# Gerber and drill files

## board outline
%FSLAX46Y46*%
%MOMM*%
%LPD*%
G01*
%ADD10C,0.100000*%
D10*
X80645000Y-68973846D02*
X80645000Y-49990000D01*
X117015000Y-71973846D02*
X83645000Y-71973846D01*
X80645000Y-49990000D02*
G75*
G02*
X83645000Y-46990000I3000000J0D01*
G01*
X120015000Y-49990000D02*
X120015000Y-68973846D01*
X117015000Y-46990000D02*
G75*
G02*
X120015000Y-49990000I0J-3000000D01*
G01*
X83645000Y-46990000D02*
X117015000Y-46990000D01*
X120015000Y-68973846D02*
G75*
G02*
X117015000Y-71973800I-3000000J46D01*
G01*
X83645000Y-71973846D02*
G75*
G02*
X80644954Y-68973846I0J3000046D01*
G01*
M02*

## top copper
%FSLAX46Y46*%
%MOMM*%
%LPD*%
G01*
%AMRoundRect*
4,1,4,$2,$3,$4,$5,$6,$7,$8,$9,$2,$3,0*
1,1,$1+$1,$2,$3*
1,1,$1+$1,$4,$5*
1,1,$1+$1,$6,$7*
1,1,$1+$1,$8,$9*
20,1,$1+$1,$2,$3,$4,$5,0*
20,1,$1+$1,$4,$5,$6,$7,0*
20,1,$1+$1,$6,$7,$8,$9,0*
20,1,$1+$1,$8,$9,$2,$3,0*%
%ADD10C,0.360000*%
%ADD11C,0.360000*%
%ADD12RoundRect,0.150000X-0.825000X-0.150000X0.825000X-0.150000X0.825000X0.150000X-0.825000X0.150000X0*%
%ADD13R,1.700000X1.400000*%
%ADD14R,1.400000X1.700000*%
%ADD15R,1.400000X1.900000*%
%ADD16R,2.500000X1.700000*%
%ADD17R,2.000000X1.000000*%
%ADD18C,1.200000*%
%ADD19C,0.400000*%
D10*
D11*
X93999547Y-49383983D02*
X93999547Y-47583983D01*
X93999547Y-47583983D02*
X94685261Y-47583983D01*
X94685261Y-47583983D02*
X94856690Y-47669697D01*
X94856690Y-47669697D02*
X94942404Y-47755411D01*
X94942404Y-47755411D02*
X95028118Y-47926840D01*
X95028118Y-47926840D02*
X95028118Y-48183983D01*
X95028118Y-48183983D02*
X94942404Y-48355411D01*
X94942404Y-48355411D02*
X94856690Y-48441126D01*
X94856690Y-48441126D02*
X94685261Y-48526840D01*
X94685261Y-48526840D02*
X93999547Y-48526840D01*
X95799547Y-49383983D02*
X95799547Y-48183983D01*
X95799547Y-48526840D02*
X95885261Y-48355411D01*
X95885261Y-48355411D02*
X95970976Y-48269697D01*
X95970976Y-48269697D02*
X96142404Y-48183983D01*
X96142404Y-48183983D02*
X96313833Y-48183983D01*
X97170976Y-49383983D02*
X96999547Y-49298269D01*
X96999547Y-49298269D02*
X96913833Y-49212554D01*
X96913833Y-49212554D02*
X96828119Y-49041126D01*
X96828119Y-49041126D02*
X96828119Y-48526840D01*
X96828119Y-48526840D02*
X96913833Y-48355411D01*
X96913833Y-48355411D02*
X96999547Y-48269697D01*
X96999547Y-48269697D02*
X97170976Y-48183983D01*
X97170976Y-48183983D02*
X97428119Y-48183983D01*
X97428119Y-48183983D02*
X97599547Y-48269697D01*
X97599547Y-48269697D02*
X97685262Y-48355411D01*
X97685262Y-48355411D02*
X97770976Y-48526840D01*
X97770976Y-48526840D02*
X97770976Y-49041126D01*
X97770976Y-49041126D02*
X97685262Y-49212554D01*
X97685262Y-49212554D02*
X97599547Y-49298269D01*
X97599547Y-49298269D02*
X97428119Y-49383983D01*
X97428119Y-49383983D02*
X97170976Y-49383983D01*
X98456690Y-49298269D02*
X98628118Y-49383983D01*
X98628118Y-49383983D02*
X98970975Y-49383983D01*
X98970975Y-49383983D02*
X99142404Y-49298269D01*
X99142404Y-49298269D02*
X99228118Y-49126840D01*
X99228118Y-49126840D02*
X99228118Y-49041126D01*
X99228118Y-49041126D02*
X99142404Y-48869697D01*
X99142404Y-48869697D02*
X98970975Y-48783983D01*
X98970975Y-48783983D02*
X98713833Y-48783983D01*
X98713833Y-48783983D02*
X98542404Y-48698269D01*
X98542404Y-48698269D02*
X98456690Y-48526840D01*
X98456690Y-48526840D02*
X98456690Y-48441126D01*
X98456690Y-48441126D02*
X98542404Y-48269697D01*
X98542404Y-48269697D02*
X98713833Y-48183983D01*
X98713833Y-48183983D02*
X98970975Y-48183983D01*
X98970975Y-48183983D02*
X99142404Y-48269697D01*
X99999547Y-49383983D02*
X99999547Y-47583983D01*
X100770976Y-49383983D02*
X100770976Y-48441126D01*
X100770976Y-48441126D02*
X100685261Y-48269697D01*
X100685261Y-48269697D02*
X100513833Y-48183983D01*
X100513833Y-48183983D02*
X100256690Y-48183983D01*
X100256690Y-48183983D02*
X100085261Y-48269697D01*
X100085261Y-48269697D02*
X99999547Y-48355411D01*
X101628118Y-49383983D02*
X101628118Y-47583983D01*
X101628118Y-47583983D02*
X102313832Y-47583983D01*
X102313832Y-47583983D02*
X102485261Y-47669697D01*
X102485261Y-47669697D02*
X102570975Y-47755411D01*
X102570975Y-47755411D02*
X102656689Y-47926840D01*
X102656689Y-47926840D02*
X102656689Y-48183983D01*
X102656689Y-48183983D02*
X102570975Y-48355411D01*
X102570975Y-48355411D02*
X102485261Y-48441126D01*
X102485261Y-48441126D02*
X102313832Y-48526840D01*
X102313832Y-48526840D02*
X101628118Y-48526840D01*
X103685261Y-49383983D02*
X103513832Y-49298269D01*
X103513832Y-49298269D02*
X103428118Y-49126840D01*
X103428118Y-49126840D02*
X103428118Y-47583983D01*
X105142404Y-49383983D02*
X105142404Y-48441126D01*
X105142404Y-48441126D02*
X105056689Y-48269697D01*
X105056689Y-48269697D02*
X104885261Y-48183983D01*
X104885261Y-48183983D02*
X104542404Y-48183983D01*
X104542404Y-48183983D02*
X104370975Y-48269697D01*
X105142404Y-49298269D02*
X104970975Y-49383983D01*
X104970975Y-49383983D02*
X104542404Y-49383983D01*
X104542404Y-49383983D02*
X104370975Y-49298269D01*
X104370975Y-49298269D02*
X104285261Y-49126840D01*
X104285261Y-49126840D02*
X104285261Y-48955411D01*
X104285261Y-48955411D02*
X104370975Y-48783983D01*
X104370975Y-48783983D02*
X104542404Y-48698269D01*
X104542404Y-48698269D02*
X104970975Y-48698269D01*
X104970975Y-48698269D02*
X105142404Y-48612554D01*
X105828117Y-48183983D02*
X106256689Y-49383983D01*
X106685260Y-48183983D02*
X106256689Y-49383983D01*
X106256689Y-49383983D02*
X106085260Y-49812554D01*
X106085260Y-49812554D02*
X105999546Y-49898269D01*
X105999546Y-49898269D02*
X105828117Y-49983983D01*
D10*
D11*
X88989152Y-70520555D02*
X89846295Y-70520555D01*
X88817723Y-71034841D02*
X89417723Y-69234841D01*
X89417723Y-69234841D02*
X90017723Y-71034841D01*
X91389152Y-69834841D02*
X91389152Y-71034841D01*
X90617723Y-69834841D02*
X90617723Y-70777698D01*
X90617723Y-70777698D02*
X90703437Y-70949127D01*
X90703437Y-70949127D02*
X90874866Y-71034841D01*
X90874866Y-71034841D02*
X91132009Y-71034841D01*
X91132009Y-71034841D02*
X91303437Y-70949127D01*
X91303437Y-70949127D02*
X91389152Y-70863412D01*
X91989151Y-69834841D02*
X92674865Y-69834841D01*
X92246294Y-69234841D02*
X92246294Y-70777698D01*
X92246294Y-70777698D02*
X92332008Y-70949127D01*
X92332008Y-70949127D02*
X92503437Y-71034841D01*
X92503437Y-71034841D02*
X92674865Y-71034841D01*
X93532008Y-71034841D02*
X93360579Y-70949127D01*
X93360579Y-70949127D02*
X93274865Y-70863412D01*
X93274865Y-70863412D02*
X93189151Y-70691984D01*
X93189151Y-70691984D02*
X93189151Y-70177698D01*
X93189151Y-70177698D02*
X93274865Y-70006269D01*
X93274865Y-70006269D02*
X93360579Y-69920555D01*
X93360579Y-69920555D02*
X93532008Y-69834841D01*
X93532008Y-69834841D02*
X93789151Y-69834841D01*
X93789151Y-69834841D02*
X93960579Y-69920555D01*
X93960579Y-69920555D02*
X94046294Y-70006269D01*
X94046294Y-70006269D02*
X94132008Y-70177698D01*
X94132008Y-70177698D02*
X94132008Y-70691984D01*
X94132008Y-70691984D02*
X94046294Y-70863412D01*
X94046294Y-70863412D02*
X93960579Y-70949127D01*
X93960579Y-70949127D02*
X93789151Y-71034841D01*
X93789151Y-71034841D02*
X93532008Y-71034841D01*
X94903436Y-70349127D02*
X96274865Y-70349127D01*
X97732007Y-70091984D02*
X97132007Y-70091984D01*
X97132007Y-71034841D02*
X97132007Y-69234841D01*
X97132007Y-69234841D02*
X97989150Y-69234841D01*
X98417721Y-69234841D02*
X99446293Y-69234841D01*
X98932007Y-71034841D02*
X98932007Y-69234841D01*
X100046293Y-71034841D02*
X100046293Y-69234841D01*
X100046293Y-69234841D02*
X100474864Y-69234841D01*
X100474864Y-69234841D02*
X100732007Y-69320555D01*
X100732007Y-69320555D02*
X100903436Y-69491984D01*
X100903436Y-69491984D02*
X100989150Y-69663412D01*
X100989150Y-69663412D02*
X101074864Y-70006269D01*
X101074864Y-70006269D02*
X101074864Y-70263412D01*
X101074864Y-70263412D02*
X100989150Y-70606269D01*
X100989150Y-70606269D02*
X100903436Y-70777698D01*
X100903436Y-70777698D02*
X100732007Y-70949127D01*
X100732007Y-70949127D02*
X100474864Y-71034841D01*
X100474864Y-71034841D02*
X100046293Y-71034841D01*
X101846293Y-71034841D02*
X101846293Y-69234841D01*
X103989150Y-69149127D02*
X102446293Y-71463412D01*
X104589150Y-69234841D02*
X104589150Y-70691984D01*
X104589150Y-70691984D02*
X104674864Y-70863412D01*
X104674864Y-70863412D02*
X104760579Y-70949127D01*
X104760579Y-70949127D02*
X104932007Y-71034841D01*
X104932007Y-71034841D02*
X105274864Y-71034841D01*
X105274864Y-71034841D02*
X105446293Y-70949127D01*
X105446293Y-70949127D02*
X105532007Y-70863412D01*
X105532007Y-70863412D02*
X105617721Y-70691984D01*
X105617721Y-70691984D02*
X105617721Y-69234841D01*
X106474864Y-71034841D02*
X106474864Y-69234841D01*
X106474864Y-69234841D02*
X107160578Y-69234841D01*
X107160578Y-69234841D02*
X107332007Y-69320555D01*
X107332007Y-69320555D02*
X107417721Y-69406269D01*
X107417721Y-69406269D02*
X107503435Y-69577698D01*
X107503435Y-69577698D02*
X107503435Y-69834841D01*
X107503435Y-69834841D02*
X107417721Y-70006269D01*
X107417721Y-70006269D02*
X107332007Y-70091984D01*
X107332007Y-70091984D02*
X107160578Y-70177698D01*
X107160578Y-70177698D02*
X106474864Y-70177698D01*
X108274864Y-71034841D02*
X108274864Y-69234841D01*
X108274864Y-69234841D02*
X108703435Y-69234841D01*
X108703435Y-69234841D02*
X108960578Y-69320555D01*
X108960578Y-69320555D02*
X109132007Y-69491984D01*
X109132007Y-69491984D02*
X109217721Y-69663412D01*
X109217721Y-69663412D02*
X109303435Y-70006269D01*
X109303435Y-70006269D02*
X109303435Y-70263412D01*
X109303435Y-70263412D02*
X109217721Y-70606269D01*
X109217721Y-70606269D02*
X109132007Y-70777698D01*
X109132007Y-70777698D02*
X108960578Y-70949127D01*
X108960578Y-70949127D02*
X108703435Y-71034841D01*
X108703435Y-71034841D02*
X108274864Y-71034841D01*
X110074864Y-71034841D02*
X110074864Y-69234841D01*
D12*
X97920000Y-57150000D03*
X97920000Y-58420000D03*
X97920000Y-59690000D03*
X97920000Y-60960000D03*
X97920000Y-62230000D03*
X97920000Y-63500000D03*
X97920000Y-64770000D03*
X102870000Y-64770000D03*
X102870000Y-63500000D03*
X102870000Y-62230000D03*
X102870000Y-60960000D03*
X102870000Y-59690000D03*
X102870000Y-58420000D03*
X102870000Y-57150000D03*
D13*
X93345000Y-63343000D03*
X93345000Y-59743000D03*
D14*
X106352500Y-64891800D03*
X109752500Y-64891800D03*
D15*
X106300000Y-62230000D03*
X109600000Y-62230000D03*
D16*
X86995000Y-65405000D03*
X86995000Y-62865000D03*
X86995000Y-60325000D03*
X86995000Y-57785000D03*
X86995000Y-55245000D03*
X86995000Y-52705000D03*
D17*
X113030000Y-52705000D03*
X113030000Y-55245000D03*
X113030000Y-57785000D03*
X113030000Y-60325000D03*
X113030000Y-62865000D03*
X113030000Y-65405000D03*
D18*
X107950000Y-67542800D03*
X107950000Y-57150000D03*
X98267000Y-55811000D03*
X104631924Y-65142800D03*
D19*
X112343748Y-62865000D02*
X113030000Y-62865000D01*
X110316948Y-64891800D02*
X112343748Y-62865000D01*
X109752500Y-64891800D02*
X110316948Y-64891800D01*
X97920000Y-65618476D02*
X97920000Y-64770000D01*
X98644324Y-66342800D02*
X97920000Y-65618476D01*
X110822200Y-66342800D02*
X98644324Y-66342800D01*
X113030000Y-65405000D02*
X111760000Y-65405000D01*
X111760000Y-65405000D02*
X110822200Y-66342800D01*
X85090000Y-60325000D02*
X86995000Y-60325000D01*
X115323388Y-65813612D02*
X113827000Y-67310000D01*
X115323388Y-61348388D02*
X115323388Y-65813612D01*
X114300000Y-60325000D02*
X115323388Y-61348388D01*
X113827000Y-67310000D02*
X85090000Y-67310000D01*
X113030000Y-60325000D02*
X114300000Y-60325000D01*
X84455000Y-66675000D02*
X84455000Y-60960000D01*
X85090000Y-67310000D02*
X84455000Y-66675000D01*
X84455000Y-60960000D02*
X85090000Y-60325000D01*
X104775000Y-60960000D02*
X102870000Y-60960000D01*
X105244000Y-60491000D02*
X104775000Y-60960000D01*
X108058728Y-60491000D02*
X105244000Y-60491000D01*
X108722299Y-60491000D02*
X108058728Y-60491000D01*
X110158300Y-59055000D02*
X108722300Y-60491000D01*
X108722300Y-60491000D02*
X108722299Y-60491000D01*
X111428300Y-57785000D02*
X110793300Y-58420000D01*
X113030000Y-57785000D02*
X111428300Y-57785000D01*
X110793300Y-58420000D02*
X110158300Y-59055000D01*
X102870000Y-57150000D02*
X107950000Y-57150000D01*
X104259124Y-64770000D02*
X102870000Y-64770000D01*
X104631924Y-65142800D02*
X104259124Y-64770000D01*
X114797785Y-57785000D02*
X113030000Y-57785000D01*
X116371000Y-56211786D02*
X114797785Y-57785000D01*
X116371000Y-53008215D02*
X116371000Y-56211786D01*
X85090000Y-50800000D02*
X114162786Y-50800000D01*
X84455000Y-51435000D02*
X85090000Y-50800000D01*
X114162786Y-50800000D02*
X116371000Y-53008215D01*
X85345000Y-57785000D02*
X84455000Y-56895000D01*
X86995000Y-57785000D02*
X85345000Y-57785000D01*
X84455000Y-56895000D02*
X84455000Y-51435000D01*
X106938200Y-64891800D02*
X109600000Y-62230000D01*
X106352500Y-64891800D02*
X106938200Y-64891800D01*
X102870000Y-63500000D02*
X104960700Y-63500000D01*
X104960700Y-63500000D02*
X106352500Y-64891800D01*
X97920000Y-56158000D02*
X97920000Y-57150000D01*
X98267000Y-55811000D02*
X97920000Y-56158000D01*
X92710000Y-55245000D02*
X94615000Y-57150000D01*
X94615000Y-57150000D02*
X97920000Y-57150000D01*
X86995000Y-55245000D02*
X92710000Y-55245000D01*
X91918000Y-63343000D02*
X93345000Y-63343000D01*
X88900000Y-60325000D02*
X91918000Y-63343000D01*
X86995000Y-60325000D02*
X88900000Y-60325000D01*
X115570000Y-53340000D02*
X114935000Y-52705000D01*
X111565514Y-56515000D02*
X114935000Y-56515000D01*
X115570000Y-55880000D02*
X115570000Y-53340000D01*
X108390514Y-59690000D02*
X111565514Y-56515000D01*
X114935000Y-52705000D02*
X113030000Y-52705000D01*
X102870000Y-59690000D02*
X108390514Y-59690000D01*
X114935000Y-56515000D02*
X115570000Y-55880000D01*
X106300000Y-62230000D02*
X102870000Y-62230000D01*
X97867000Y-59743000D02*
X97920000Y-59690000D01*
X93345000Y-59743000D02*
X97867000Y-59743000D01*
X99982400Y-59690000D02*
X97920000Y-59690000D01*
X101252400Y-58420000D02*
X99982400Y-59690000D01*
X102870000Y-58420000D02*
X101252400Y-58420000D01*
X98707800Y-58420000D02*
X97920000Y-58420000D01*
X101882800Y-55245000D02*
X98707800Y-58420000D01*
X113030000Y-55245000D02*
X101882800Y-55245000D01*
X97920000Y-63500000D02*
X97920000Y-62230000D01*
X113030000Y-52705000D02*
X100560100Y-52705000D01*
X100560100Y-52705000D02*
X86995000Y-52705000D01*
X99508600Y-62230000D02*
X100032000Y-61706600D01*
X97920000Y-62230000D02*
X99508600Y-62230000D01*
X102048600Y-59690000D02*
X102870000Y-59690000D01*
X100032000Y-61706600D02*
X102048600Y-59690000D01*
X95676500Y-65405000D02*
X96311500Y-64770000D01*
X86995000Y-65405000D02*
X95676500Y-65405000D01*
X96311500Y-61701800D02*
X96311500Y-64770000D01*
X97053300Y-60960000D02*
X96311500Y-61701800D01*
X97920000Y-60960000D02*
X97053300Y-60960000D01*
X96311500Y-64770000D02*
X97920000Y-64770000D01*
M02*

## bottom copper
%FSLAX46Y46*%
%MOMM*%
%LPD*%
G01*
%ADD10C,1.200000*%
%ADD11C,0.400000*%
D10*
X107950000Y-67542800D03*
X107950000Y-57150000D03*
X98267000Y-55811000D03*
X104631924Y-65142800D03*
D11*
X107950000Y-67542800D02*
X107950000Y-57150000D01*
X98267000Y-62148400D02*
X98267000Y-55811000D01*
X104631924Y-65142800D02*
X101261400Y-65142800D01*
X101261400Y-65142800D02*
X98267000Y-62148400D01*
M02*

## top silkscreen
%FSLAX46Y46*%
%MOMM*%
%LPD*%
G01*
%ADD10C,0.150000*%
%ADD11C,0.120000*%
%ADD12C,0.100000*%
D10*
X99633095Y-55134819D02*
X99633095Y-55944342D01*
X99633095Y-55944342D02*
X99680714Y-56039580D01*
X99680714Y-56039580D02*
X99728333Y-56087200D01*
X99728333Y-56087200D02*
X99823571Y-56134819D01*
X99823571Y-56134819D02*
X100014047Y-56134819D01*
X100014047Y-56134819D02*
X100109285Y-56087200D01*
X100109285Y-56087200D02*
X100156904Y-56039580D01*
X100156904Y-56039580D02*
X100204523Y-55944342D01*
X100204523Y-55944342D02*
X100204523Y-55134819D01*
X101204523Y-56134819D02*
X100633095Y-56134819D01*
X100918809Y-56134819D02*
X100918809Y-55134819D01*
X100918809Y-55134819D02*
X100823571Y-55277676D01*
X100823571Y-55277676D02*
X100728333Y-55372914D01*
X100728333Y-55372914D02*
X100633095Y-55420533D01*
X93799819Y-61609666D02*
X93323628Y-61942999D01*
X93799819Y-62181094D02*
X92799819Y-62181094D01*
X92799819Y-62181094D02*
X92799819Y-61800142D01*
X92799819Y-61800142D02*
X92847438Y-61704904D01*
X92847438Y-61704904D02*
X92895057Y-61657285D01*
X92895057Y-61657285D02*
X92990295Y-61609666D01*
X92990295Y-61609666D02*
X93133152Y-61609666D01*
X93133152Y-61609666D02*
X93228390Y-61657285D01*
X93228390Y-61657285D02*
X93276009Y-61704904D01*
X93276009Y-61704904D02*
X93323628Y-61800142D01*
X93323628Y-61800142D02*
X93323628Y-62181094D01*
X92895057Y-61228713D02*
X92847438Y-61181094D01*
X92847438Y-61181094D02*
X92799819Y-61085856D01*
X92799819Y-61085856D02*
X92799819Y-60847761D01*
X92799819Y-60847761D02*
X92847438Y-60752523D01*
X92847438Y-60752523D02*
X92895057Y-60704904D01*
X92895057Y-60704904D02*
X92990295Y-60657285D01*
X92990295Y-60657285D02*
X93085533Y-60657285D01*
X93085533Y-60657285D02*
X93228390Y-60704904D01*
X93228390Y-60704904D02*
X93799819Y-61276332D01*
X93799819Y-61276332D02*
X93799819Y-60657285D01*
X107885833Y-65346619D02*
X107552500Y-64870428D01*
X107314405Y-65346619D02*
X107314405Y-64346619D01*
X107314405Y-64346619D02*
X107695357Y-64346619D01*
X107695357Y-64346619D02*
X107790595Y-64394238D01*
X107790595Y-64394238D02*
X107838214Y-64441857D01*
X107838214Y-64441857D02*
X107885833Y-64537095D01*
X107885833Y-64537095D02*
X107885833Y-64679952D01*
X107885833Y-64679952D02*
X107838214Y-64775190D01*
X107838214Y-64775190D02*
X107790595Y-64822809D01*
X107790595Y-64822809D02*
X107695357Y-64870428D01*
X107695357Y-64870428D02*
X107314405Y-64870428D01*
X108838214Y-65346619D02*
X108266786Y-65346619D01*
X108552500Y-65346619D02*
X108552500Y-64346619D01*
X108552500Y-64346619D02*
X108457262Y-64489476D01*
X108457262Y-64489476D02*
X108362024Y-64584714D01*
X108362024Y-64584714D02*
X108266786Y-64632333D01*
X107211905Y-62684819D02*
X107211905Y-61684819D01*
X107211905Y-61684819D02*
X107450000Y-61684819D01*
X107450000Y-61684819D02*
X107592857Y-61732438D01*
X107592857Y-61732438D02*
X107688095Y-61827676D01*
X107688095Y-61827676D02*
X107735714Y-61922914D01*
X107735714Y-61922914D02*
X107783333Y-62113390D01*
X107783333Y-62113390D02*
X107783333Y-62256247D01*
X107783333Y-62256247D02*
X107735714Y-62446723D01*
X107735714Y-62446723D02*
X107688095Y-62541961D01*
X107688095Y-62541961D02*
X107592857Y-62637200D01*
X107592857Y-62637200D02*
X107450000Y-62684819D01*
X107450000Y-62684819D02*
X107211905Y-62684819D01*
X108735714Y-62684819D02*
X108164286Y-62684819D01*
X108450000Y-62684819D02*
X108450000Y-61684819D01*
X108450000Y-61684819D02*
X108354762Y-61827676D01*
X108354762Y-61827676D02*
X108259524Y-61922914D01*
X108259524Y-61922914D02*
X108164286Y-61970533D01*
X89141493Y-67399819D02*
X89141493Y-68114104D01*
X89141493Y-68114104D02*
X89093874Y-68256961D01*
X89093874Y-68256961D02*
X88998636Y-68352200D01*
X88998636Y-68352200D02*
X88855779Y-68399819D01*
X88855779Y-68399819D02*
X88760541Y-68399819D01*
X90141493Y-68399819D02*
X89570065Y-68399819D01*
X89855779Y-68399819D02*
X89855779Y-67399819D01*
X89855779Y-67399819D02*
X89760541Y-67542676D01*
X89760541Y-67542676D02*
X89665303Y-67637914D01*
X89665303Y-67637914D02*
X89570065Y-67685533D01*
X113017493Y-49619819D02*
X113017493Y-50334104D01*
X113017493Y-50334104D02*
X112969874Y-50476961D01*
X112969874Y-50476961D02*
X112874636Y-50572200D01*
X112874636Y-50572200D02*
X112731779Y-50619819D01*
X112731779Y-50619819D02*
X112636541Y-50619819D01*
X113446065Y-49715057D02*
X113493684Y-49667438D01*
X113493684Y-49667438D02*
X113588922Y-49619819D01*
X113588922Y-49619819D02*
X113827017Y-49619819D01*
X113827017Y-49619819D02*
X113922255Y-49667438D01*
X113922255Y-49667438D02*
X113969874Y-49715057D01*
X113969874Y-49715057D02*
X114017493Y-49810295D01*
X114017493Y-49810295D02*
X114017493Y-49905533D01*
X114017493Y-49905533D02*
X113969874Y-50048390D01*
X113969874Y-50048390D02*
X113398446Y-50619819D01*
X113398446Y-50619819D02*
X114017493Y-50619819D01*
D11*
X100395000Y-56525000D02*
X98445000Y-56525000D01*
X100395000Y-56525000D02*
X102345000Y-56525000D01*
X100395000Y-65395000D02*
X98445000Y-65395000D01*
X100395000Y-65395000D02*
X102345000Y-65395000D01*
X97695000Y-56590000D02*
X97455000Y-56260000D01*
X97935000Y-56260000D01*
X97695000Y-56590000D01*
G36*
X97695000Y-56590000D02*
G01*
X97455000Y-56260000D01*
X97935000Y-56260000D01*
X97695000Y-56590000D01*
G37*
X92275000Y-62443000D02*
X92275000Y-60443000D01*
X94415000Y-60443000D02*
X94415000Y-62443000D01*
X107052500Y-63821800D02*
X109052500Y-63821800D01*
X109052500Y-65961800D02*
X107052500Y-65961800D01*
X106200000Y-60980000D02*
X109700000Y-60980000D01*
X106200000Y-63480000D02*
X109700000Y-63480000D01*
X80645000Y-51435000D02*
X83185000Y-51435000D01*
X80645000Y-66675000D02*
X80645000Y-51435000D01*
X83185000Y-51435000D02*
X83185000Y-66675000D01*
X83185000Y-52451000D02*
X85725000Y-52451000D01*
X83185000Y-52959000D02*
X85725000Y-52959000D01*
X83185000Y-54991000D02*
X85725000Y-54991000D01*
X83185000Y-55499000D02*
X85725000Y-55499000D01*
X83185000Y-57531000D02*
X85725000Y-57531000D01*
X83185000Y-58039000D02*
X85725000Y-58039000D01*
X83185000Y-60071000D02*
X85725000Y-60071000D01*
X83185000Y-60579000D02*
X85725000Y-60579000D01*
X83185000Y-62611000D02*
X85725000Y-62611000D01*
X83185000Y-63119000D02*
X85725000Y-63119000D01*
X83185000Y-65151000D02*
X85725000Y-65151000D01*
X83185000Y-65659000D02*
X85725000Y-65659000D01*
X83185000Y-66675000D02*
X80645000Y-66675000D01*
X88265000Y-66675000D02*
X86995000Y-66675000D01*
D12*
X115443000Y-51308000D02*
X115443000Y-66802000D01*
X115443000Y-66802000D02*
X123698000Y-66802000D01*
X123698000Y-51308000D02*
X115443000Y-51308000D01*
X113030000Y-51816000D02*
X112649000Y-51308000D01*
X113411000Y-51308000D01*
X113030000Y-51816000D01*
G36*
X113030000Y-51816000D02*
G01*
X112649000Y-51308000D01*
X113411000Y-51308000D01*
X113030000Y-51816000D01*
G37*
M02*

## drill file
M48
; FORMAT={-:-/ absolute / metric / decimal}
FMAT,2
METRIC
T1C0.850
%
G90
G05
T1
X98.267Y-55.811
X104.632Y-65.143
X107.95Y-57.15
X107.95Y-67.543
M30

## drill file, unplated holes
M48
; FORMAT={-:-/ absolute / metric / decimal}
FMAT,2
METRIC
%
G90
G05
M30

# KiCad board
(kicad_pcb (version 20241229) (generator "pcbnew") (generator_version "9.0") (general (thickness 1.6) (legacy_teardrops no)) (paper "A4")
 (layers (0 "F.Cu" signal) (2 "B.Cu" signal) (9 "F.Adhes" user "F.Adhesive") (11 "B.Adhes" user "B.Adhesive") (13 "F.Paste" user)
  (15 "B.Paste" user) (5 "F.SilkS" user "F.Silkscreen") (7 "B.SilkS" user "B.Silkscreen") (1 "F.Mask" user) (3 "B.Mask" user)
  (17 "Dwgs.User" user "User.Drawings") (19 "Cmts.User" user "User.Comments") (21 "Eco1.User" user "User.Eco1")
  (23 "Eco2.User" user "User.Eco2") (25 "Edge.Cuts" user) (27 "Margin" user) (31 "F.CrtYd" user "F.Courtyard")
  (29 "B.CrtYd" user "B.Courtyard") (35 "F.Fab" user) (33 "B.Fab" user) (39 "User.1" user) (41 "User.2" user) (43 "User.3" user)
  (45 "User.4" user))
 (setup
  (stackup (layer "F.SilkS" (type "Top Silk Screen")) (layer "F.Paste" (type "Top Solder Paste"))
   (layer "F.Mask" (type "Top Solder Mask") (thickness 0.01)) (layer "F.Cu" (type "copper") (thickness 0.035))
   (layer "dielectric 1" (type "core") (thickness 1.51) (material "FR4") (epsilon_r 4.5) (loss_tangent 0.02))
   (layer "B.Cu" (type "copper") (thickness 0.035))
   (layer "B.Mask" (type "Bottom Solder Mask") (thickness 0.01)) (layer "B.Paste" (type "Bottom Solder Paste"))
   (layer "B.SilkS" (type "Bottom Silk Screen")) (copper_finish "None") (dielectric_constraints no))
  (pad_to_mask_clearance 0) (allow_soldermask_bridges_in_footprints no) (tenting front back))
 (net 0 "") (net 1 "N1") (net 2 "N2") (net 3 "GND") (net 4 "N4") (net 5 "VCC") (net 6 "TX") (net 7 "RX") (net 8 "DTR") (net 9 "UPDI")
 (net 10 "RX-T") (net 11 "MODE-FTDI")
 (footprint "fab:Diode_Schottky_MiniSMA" (layer "F.Cu") (at 107.95 62.23)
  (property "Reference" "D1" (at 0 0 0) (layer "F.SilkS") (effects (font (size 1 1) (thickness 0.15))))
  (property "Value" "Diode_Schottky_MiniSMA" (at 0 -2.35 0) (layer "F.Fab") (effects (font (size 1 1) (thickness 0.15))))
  (fp_line (start -1.75 -1.25) (end 1.75 -1.25) (stroke (width 0.12) (type solid)) (layer "F.SilkS"))
  (fp_line (start -1.75 1.25) (end 1.75 1.25) (stroke (width 0.12) (type solid)) (layer "F.SilkS"))
  (pad "1" smd rect (at -1.65 0) (size 1.4 1.9) (layers "F.Cu" "F.Mask" "F.Paste") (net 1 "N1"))
  (pad "2" smd rect (at 1.65 0) (size 1.4 1.9) (layers "F.Cu" "F.Mask" "F.Paste") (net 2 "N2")))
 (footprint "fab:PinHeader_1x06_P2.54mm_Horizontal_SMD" (layer "F.Cu") (at 86.995 65.405 180)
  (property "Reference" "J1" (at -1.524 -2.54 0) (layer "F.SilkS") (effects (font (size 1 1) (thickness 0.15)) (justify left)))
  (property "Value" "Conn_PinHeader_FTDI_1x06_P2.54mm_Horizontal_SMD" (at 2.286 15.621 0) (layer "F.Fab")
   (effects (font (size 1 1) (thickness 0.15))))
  (fp_line (start 6.35 13.97) (end 3.81 13.97) (stroke (width 0.12) (type solid)) (layer "F.SilkS"))
  (fp_line (start 6.35 -1.27) (end 6.35 13.97) (stroke (width 0.12) (type solid)) (layer "F.SilkS"))
  (fp_line (start 3.81 13.97) (end 3.81 -1.27) (stroke (width 0.12) (type solid)) (layer "F.SilkS"))
  (fp_line (start 3.81 12.954) (end 1.27 12.954) (stroke (width 0.12) (type solid)) (layer "F.SilkS"))
  (fp_line (start 3.81 12.446) (end 1.27 12.446) (stroke (width 0.12) (type solid)) (layer "F.SilkS"))
  (fp_line (start 3.81 10.414) (end 1.27 10.414) (stroke (width 0.12) (type solid)) (layer "F.SilkS"))
  (fp_line (start 3.81 9.906) (end 1.27 9.906) (stroke (width 0.12) (type solid)) (layer "F.SilkS"))
  (fp_line (start 3.81 7.874) (end 1.27 7.874) (stroke (width 0.12) (type solid)) (layer "F.SilkS"))
  (fp_line (start 3.81 7.366) (end 1.27 7.366) (stroke (width 0.12) (type solid)) (layer "F.SilkS"))
  (fp_line (start 3.81 5.334) (end 1.27 5.334) (stroke (width 0.12) (type solid)) (layer "F.SilkS"))
  (fp_line (start 3.81 4.826) (end 1.27 4.826) (stroke (width 0.12) (type solid)) (layer "F.SilkS"))
  (fp_line (start 3.81 2.794) (end 1.27 2.794) (stroke (width 0.12) (type solid)) (layer "F.SilkS"))
  (fp_line (start 3.81 2.286) (end 1.27 2.286) (stroke (width 0.12) (type solid)) (layer "F.SilkS"))
  (fp_line (start 3.81 0.254) (end 1.27 0.254) (stroke (width 0.12) (type solid)) (layer "F.SilkS"))
  (fp_line (start 3.81 -0.254) (end 1.27 -0.254) (stroke (width 0.12) (type solid)) (layer "F.SilkS"))
  (fp_line (start 3.81 -1.27) (end 6.35 -1.27) (stroke (width 0.12) (type solid)) (layer "F.SilkS"))
  (fp_line (start -1.27 -1.27) (end 0 -1.27) (stroke (width 0.12) (type solid)) (layer "F.SilkS"))
  (pad "1" smd rect (at 0 0 180) (size 2.5 1.7) (layers "F.Cu" "F.Mask" "F.Paste") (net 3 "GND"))
  (pad "2" smd rect (at 0 2.54 180) (size 2.5 1.7) (layers "F.Cu" "F.Mask" "F.Paste") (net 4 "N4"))
  (pad "3" smd rect (at 0 5.08 180) (size 2.5 1.7) (layers "F.Cu" "F.Mask" "F.Paste") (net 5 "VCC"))
  (pad "4" smd rect (at 0 7.62 180) (size 2.5 1.7) (layers "F.Cu" "F.Mask" "F.Paste") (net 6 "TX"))
  (pad "5" smd rect (at 0 10.16 180) (size 2.5 1.7) (layers "F.Cu" "F.Mask" "F.Paste") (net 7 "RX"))
  (pad "6" smd rect (at 0 12.7 180) (size 2.5 1.7) (layers "F.Cu" "F.Mask" "F.Paste") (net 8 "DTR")))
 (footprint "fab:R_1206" (layer "F.Cu") (at 108.0525 64.8918)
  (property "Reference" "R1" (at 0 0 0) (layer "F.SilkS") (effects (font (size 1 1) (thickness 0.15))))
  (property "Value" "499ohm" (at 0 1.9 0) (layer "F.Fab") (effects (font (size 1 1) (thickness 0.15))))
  (fp_line (start -1 -1.07) (end 1 -1.07) (stroke (width 0.12) (type solid)) (layer "F.SilkS"))
  (fp_line (start 1 1.07) (end -1 1.07) (stroke (width 0.12) (type solid)) (layer "F.SilkS"))
  (pad "1" smd rect (at -1.7 0) (size 1.4 1.7) (layers "F.Cu" "F.Mask" "F.Paste") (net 2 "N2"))
  (pad "2" smd rect (at 1.7 0) (size 1.4 1.7) (layers "F.Cu" "F.Mask" "F.Paste") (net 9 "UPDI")))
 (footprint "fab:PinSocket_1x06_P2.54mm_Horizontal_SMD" (layer "F.Cu") (at 113.03 52.705)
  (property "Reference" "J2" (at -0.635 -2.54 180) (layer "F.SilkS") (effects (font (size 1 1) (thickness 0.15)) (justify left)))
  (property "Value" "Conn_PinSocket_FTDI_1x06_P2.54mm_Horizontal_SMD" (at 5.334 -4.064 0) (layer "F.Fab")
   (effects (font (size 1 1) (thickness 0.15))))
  (fp_line (start 2.413 -1.397) (end 2.413 14.097) (stroke (width 0.1) (type default)) (layer "F.SilkS"))
  (fp_line (start 2.413 14.097) (end 10.668 14.097) (stroke (width 0.1) (type default)) (layer "F.SilkS"))
  (fp_line (start 10.668 -1.397) (end 2.413 -1.397) (stroke (width 0.1) (type default)) (layer "F.SilkS"))
  (fp_poly (pts (xy 0 -0.889) (xy -0.381 -1.397) (xy 0.381 -1.397)) (stroke (width 0.1) (type solid)) (fill yes) (layer "F.SilkS"))
  (pad "1" smd rect (at 0 0) (size 2 1) (layers "F.Cu" "F.Mask" "F.Paste") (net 8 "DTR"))
  (pad "2" smd rect (at 0 2.54) (size 2 1) (layers "F.Cu" "F.Mask" "F.Paste") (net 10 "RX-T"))
  (pad "3" smd rect (at 0 5.08) (size 2 1) (layers "F.Cu" "F.Mask" "F.Paste") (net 6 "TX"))
  (pad "4" smd rect (at 0 7.62) (size 2 1) (layers "F.Cu" "F.Mask" "F.Paste") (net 5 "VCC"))
  (pad "5" smd rect (at 0 10.16) (size 2 1) (layers "F.Cu" "F.Mask" "F.Paste") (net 9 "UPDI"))
  (pad "6" smd rect (at 0 12.7) (size 2 1) (layers "F.Cu" "F.Mask" "F.Paste") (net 3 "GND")))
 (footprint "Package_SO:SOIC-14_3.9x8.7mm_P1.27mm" (layer "F.Cu") (at 100.395 60.96)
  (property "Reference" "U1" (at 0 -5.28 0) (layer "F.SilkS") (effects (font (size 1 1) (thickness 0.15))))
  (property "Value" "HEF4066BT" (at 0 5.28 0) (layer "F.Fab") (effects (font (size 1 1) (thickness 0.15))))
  (fp_line (start 0 -4.435) (end -1.95 -4.435) (stroke (width 0.12) (type solid)) (layer "F.SilkS"))
  (fp_line (start 0 -4.435) (end 1.95 -4.435) (stroke (width 0.12) (type solid)) (layer "F.SilkS"))
  (fp_line (start 0 4.435) (end -1.95 4.435) (stroke (width 0.12) (type solid)) (layer "F.SilkS"))
  (fp_line (start 0 4.435) (end 1.95 4.435) (stroke (width 0.12) (type solid)) (layer "F.SilkS"))
  (fp_poly
   (pts (xy -2.7 -4.37) (xy -2.94 -4.7) (xy -2.46 -4.7) (xy -2.7 -4.37)) (stroke (width 0.12) (type solid)) (fill yes) (layer "F.SilkS"))
  (pad "1" smd roundrect (at -2.475 -3.81) (size 1.95 0.6) (layers "F.Cu" "F.Mask" "F.Paste") (roundrect_rratio 0.25) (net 7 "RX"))
  (pad "2" smd roundrect (at -2.475 -2.54) (size 1.95 0.6) (layers "F.Cu" "F.Mask" "F.Paste") (roundrect_rratio 0.25) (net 10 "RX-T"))
  (pad "3" smd roundrect (at -2.475 -1.27) (size 1.95 0.6) (layers "F.Cu" "F.Mask" "F.Paste") (roundrect_rratio 0.25) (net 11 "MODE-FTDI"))
  (pad "4" smd roundrect (at -2.475 0) (size 1.95 0.6) (layers "F.Cu" "F.Mask" "F.Paste") (roundrect_rratio 0.25) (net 3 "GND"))
  (pad "5" smd roundrect (at -2.475 1.27) (size 1.95 0.6) (layers "F.Cu" "F.Mask" "F.Paste") (roundrect_rratio 0.25) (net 8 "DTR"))
  (pad "6" smd roundrect (at -2.475 2.54) (size 1.95 0.6) (layers "F.Cu" "F.Mask" "F.Paste") (roundrect_rratio 0.25) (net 8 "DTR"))
  (pad "7" smd roundrect (at -2.475 3.81) (size 1.95 0.6) (layers "F.Cu" "F.Mask" "F.Paste") (roundrect_rratio 0.25) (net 3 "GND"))
  (pad "8" smd roundrect (at 2.475 3.81) (size 1.95 0.6) (layers "F.Cu" "F.Mask" "F.Paste") (roundrect_rratio 0.25) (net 7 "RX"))
  (pad "9" smd roundrect (at 2.475 2.54) (size 1.95 0.6) (layers "F.Cu" "F.Mask" "F.Paste") (roundrect_rratio 0.25) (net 2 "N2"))
  (pad "10" smd roundrect (at 2.475 1.27) (size 1.95 0.6) (layers "F.Cu" "F.Mask" "F.Paste") (roundrect_rratio 0.25) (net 1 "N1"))
  (pad "11" smd roundrect (at 2.475 0) (size 1.95 0.6) (layers "F.Cu" "F.Mask" "F.Paste") (roundrect_rratio 0.25) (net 6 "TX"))
  (pad "12" smd roundrect (at 2.475 -1.27) (size 1.95 0.6) (layers "F.Cu" "F.Mask" "F.Paste") (roundrect_rratio 0.25) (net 8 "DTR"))
  (pad "13" smd roundrect (at 2.475 -2.54) (size 1.95 0.6) (layers "F.Cu" "F.Mask" "F.Paste") (roundrect_rratio 0.25) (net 11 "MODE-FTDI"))
  (pad "14" smd roundrect (at 2.475 -3.81) (size 1.95 0.6) (layers "F.Cu" "F.Mask" "F.Paste") (roundrect_rratio 0.25) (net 5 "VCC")))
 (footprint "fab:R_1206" (layer "F.Cu") (at 93.345 61.443 -90)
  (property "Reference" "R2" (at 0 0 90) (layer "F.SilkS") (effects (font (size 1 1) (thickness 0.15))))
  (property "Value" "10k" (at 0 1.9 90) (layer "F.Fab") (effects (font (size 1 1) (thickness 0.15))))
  (fp_line (start 1 1.07) (end -1 1.07) (stroke (width 0.12) (type solid)) (layer "F.SilkS"))
  (fp_line (start -1 -1.07) (end 1 -1.07) (stroke (width 0.12) (type solid)) (layer "F.SilkS"))
  (pad "1" smd rect (at -1.7 0 270) (size 1.4 1.7) (layers "F.Cu" "F.Mask" "F.Paste") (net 11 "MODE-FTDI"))
  (pad "2" smd rect (at 1.9 0 270) (size 1.4 1.7) (layers "F.Cu" "F.Mask" "F.Paste") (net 5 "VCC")))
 (gr_line (start 80.645 68.973846) (end 80.645 49.99) (stroke (width 0.1) (type default)) (layer "Edge.Cuts"))
 (gr_line (start 117.015 71.973846) (end 83.645 71.973846) (stroke (width 0.1) (type default)) (layer "Edge.Cuts"))
 (gr_arc (start 80.645 49.99) (mid 81.52368 47.86868) (end 83.645 46.99) (stroke (width 0.1) (type default)) (layer "Edge.Cuts"))
 (gr_line (start 120.015 49.99) (end 120.015 68.973846) (stroke (width 0.1) (type default)) (layer "Edge.Cuts"))
 (gr_arc (start 117.015 46.99) (mid 119.13632 47.86868) (end 120.015 49.99) (stroke (width 0.1) (type default)) (layer "Edge.Cuts"))
 (gr_line (start 83.645 46.99) (end 117.015 46.99) (stroke (width 0.1) (type default)) (layer "Edge.Cuts"))
 (gr_arc (start 120.015 68.973846) (mid 119.13632 71.095166) (end 117.015 71.973846) (stroke (width 0.1) (type default)) (layer "Edge.Cuts"))
 (gr_arc (start 83.645 71.973846) (mid 81.523678 71.095167) (end 80.645 68.973846) (stroke (width 0.1) (type default)) (layer "Edge.Cuts"))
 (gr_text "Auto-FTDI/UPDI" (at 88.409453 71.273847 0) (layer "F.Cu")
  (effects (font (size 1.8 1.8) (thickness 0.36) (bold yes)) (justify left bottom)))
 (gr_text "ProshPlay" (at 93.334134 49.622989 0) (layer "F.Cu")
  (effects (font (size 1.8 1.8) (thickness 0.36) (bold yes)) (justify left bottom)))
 (segment (start 104.9607 63.5) (end 106.3525 64.8918) (width 0.4) (layer "F.Cu") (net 2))
 (segment (start 106.9382 64.8918) (end 109.6 62.23) (width 0.4) (layer "F.Cu") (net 2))
 (segment (start 106.3525 64.8918) (end 106.9382 64.8918) (width 0.4) (layer "F.Cu") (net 2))
 (segment (start 102.87 63.5) (end 104.9607 63.5) (width 0.4) (layer "F.Cu") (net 2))
 (segment (start 115.323388 65.813612) (end 113.827 67.31) (width 0.4) (layer "F.Cu") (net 5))
 (segment (start 113.03 60.325) (end 114.3 60.325) (width 0.4) (layer "F.Cu") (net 5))
 (segment (start 114.3 60.325) (end 115.323388 61.348388) (width 0.4) (layer "F.Cu") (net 5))
 (segment (start 85.09 67.31) (end 84.455 66.675) (width 0.4) (layer "F.Cu") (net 5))
 (segment (start 91.918 63.343) (end 93.345 63.343) (width 0.4) (layer "F.Cu") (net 5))
 (segment (start 113.827 67.31) (end 85.09 67.31) (width 0.4) (layer "F.Cu") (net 5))
 (segment (start 85.09 60.325) (end 86.995 60.325) (width 0.4) (layer "F.Cu") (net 5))
 (segment (start 84.455 66.675) (end 84.455 60.96) (width 0.4) (layer "F.Cu") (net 5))
 (segment (start 115.323388 61.348388) (end 115.323388 65.813612) (width 0.4) (layer "F.Cu") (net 5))
 (segment (start 84.455 60.96) (end 85.09 60.325) (width 0.4) (layer "F.Cu") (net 5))
 (segment (start 88.9 60.325) (end 91.918 63.343) (width 0.4) (layer "F.Cu") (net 5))
 (segment (start 86.995 60.325) (end 88.9 60.325) (width 0.4) (layer "F.Cu") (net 5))
 (segment (start 102.87 57.15) (end 107.95 57.15) (width 0.4) (layer "F.Cu") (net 5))
 (via (at 107.95 57.15) (size 1.2) (drill 0.85) (layers "F.Cu" "B.Cu") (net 5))
 (via (at 107.95 67.5428) (size 1.2) (drill 0.85) (layers "F.Cu" "B.Cu") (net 5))
 (segment (start 107.95 67.5428) (end 107.95 57.15) (width 0.4) (layer "B.Cu") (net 5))
 (segment (start 113.03 65.405) (end 111.76 65.405) (width 0.4) (layer "F.Cu") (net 3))
 (segment (start 97.0533 60.96) (end 96.3115 61.7018) (width 0.4) (layer "F.Cu") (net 3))
 (segment (start 97.92 60.96) (end 97.0533 60.96) (width 0.4) (layer "F.Cu") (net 3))
 (segment (start 110.8222 66.3428) (end 98.644324 66.3428) (width 0.4) (layer "F.Cu") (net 3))
 (segment (start 111.76 65.405) (end 110.8222 66.3428) (width 0.4) (layer "F.Cu") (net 3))
 (segment (start 98.644324 66.3428) (end 97.92 65.618476) (width 0.4) (layer "F.Cu") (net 3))
 (segment (start 95.6765 65.405) (end 96.3115 64.77) (width 0.4) (layer "F.Cu") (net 3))
 (segment (start 96.3115 61.7018) (end 96.3115 64.77) (width 0.4) (layer "F.Cu") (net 3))
 (segment (start 96.3115 64.77) (end 97.92 64.77) (width 0.4) (layer "F.Cu") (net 3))
 (segment (start 97.92 65.618476) (end 97.92 64.77) (width 0.4) (layer "F.Cu") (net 3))
 (segment (start 86.995 65.405) (end 95.6765 65.405) (width 0.4) (layer "F.Cu") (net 3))
 (segment (start 102.87 59.69) (end 108.390514 59.69) (width 0.4) (layer "F.Cu") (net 8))
 (segment (start 114.935 52.705) (end 113.03 52.705) (width 0.4) (layer "F.Cu") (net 8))
 (segment (start 100.5601 52.705) (end 86.995 52.705) (width 0.4) (layer "F.Cu") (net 8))
 (segment (start 108.390514 59.69) (end 111.565514 56.515) (width 0.4) (layer "F.Cu") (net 8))
 (segment (start 113.03 52.705) (end 100.5601 52.705) (width 0.4) (layer "F.Cu") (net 8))
 (segment (start 115.57 53.34) (end 114.935 52.705) (width 0.4) (layer "F.Cu") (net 8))
 (segment (start 111.565514 56.515) (end 114.935 56.515) (width 0.4) (layer "F.Cu") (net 8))
 (segment (start 114.935 56.515) (end 115.57 55.88) (width 0.4) (layer "F.Cu") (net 8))
 (segment (start 100.032 61.7066) (end 102.0486 59.69) (width 0.4) (layer "F.Cu") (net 8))
 (segment (start 97.92 62.23) (end 99.5086 62.23) (width 0.4) (layer "F.Cu") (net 8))
 (segment (start 97.92 63.5) (end 97.92 62.23) (width 0.4) (layer "F.Cu") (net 8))
 (segment (start 115.57 55.88) (end 115.57 53.34) (width 0.4) (layer "F.Cu") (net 8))
 (segment (start 99.5086 62.23) (end 100.032 61.7066) (width 0.4) (layer "F.Cu") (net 8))
 (segment (start 102.0486 59.69) (end 102.87 59.69) (width 0.4) (layer "F.Cu") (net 8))
 (segment (start 104.259124 64.77) (end 102.87 64.77) (width 0.4) (layer "F.Cu") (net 7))
 (segment (start 97.92 56.158) (end 97.92 57.15) (width 0.4) (layer "F.Cu") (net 7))
 (segment (start 86.995 55.245) (end 92.71 55.245) (width 0.4) (layer "F.Cu") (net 7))
 (segment (start 98.267 55.811) (end 97.92 56.158) (width 0.4) (layer "F.Cu") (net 7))
 (segment (start 92.71 55.245) (end 94.615 57.15) (width 0.4) (layer "F.Cu") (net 7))
 (segment (start 104.631924 65.1428) (end 104.259124 64.77) (width 0.4) (layer "F.Cu") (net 7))
 (segment (start 94.615 57.15) (end 97.92 57.15) (width 0.4) (layer "F.Cu") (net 7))
 (via (at 104.631924 65.1428) (size 1.2) (drill 0.85) (layers "F.Cu" "B.Cu") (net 7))
 (via (at 98.267 55.811) (size 1.2) (drill 0.85) (layers "F.Cu" "B.Cu") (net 7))
 (segment (start 98.267 62.1484) (end 98.267 55.811) (width 0.4) (layer "B.Cu") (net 7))
 (segment (start 101.2614 65.1428) (end 98.267 62.1484) (width 0.4) (layer "B.Cu") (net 7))
 (segment (start 104.631924 65.1428) (end 101.2614 65.1428) (width 0.4) (layer "B.Cu") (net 7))
 (segment (start 104.775 60.96) (end 102.87 60.96) (width 0.4) (layer "F.Cu") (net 6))
 (segment (start 85.09 50.8) (end 114.162786 50.8) (width 0.4) (layer "F.Cu") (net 6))
 (segment (start 86.995 57.785) (end 85.345 57.785) (width 0.4) (layer "F.Cu") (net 6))
 (segment (start 110.1583 59.055) (end 108.7223 60.491) (width 0.4) (layer "F.Cu") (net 6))
 (segment (start 113.03 57.785) (end 111.4283 57.785) (width 0.4) (layer "F.Cu") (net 6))
 (segment (start 116.371 53.008215) (end 116.371 56.211786) (width 0.4) (layer "F.Cu") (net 6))
 (segment (start 108.722299 60.491) (end 108.058728 60.491) (width 0.4) (layer "F.Cu") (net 6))
 (segment (start 108.7223 60.491) (end 108.722299 60.491) (width 0.4) (layer "F.Cu") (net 6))
 (segment (start 114.162786 50.8) (end 116.371 53.008215) (width 0.4) (layer "F.Cu") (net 6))
 (segment (start 114.797785 57.785) (end 113.03 57.785) (width 0.4) (layer "F.Cu") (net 6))
 (segment (start 108.058728 60.491) (end 105.244 60.491) (width 0.4) (layer "F.Cu") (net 6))
 (segment (start 111.4283 57.785) (end 110.7933 58.42) (width 0.4) (layer "F.Cu") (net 6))
 (segment (start 84.455 56.895) (end 84.455 51.435) (width 0.4) (layer "F.Cu") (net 6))
 (segment (start 116.371 56.211786) (end 114.797785 57.785) (width 0.4) (layer "F.Cu") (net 6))
 (segment (start 110.7933 58.42) (end 110.1583 59.055) (width 0.4) (layer "F.Cu") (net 6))
 (segment (start 105.244 60.491) (end 104.775 60.96) (width 0.4) (layer "F.Cu") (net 6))
 (segment (start 85.345 57.785) (end 84.455 56.895) (width 0.4) (layer "F.Cu") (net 6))
 (segment (start 84.455 51.435) (end 85.09 50.8) (width 0.4) (layer "F.Cu") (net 6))
 (segment (start 113.03 55.245) (end 101.8828 55.245) (width 0.4) (layer "F.Cu") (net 10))
 (segment (start 98.7078 58.42) (end 97.92 58.42) (width 0.4) (layer "F.Cu") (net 10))
 (segment (start 101.8828 55.245) (end 98.7078 58.42) (width 0.4) (layer "F.Cu") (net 10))
 (segment (start 109.7525 64.8918) (end 110.316948 64.8918) (width 0.4) (layer "F.Cu") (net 9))
 (segment (start 110.316948 64.8918) (end 112.343748 62.865) (width 0.4) (layer "F.Cu") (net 9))
 (segment (start 112.343748 62.865) (end 113.03 62.865) (width 0.4) (layer "F.Cu") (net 9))
 (segment (start 102.87 58.42) (end 101.2524 58.42) (width 0.4) (layer "F.Cu") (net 11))
 (segment (start 101.2524 58.42) (end 99.9824 59.69) (width 0.4) (layer "F.Cu") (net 11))
 (segment (start 99.9824 59.69) (end 97.92 59.69) (width 0.4) (layer "F.Cu") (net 11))
 (segment (start 93.345 59.743) (end 97.867 59.743) (width 0.4) (layer "F.Cu") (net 11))
 (segment (start 97.867 59.743) (end 97.92 59.69) (width 0.4) (layer "F.Cu") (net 11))
 (segment (start 106.3 62.23) (end 102.87 62.23) (width 0.4) (layer "F.Cu") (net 1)))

